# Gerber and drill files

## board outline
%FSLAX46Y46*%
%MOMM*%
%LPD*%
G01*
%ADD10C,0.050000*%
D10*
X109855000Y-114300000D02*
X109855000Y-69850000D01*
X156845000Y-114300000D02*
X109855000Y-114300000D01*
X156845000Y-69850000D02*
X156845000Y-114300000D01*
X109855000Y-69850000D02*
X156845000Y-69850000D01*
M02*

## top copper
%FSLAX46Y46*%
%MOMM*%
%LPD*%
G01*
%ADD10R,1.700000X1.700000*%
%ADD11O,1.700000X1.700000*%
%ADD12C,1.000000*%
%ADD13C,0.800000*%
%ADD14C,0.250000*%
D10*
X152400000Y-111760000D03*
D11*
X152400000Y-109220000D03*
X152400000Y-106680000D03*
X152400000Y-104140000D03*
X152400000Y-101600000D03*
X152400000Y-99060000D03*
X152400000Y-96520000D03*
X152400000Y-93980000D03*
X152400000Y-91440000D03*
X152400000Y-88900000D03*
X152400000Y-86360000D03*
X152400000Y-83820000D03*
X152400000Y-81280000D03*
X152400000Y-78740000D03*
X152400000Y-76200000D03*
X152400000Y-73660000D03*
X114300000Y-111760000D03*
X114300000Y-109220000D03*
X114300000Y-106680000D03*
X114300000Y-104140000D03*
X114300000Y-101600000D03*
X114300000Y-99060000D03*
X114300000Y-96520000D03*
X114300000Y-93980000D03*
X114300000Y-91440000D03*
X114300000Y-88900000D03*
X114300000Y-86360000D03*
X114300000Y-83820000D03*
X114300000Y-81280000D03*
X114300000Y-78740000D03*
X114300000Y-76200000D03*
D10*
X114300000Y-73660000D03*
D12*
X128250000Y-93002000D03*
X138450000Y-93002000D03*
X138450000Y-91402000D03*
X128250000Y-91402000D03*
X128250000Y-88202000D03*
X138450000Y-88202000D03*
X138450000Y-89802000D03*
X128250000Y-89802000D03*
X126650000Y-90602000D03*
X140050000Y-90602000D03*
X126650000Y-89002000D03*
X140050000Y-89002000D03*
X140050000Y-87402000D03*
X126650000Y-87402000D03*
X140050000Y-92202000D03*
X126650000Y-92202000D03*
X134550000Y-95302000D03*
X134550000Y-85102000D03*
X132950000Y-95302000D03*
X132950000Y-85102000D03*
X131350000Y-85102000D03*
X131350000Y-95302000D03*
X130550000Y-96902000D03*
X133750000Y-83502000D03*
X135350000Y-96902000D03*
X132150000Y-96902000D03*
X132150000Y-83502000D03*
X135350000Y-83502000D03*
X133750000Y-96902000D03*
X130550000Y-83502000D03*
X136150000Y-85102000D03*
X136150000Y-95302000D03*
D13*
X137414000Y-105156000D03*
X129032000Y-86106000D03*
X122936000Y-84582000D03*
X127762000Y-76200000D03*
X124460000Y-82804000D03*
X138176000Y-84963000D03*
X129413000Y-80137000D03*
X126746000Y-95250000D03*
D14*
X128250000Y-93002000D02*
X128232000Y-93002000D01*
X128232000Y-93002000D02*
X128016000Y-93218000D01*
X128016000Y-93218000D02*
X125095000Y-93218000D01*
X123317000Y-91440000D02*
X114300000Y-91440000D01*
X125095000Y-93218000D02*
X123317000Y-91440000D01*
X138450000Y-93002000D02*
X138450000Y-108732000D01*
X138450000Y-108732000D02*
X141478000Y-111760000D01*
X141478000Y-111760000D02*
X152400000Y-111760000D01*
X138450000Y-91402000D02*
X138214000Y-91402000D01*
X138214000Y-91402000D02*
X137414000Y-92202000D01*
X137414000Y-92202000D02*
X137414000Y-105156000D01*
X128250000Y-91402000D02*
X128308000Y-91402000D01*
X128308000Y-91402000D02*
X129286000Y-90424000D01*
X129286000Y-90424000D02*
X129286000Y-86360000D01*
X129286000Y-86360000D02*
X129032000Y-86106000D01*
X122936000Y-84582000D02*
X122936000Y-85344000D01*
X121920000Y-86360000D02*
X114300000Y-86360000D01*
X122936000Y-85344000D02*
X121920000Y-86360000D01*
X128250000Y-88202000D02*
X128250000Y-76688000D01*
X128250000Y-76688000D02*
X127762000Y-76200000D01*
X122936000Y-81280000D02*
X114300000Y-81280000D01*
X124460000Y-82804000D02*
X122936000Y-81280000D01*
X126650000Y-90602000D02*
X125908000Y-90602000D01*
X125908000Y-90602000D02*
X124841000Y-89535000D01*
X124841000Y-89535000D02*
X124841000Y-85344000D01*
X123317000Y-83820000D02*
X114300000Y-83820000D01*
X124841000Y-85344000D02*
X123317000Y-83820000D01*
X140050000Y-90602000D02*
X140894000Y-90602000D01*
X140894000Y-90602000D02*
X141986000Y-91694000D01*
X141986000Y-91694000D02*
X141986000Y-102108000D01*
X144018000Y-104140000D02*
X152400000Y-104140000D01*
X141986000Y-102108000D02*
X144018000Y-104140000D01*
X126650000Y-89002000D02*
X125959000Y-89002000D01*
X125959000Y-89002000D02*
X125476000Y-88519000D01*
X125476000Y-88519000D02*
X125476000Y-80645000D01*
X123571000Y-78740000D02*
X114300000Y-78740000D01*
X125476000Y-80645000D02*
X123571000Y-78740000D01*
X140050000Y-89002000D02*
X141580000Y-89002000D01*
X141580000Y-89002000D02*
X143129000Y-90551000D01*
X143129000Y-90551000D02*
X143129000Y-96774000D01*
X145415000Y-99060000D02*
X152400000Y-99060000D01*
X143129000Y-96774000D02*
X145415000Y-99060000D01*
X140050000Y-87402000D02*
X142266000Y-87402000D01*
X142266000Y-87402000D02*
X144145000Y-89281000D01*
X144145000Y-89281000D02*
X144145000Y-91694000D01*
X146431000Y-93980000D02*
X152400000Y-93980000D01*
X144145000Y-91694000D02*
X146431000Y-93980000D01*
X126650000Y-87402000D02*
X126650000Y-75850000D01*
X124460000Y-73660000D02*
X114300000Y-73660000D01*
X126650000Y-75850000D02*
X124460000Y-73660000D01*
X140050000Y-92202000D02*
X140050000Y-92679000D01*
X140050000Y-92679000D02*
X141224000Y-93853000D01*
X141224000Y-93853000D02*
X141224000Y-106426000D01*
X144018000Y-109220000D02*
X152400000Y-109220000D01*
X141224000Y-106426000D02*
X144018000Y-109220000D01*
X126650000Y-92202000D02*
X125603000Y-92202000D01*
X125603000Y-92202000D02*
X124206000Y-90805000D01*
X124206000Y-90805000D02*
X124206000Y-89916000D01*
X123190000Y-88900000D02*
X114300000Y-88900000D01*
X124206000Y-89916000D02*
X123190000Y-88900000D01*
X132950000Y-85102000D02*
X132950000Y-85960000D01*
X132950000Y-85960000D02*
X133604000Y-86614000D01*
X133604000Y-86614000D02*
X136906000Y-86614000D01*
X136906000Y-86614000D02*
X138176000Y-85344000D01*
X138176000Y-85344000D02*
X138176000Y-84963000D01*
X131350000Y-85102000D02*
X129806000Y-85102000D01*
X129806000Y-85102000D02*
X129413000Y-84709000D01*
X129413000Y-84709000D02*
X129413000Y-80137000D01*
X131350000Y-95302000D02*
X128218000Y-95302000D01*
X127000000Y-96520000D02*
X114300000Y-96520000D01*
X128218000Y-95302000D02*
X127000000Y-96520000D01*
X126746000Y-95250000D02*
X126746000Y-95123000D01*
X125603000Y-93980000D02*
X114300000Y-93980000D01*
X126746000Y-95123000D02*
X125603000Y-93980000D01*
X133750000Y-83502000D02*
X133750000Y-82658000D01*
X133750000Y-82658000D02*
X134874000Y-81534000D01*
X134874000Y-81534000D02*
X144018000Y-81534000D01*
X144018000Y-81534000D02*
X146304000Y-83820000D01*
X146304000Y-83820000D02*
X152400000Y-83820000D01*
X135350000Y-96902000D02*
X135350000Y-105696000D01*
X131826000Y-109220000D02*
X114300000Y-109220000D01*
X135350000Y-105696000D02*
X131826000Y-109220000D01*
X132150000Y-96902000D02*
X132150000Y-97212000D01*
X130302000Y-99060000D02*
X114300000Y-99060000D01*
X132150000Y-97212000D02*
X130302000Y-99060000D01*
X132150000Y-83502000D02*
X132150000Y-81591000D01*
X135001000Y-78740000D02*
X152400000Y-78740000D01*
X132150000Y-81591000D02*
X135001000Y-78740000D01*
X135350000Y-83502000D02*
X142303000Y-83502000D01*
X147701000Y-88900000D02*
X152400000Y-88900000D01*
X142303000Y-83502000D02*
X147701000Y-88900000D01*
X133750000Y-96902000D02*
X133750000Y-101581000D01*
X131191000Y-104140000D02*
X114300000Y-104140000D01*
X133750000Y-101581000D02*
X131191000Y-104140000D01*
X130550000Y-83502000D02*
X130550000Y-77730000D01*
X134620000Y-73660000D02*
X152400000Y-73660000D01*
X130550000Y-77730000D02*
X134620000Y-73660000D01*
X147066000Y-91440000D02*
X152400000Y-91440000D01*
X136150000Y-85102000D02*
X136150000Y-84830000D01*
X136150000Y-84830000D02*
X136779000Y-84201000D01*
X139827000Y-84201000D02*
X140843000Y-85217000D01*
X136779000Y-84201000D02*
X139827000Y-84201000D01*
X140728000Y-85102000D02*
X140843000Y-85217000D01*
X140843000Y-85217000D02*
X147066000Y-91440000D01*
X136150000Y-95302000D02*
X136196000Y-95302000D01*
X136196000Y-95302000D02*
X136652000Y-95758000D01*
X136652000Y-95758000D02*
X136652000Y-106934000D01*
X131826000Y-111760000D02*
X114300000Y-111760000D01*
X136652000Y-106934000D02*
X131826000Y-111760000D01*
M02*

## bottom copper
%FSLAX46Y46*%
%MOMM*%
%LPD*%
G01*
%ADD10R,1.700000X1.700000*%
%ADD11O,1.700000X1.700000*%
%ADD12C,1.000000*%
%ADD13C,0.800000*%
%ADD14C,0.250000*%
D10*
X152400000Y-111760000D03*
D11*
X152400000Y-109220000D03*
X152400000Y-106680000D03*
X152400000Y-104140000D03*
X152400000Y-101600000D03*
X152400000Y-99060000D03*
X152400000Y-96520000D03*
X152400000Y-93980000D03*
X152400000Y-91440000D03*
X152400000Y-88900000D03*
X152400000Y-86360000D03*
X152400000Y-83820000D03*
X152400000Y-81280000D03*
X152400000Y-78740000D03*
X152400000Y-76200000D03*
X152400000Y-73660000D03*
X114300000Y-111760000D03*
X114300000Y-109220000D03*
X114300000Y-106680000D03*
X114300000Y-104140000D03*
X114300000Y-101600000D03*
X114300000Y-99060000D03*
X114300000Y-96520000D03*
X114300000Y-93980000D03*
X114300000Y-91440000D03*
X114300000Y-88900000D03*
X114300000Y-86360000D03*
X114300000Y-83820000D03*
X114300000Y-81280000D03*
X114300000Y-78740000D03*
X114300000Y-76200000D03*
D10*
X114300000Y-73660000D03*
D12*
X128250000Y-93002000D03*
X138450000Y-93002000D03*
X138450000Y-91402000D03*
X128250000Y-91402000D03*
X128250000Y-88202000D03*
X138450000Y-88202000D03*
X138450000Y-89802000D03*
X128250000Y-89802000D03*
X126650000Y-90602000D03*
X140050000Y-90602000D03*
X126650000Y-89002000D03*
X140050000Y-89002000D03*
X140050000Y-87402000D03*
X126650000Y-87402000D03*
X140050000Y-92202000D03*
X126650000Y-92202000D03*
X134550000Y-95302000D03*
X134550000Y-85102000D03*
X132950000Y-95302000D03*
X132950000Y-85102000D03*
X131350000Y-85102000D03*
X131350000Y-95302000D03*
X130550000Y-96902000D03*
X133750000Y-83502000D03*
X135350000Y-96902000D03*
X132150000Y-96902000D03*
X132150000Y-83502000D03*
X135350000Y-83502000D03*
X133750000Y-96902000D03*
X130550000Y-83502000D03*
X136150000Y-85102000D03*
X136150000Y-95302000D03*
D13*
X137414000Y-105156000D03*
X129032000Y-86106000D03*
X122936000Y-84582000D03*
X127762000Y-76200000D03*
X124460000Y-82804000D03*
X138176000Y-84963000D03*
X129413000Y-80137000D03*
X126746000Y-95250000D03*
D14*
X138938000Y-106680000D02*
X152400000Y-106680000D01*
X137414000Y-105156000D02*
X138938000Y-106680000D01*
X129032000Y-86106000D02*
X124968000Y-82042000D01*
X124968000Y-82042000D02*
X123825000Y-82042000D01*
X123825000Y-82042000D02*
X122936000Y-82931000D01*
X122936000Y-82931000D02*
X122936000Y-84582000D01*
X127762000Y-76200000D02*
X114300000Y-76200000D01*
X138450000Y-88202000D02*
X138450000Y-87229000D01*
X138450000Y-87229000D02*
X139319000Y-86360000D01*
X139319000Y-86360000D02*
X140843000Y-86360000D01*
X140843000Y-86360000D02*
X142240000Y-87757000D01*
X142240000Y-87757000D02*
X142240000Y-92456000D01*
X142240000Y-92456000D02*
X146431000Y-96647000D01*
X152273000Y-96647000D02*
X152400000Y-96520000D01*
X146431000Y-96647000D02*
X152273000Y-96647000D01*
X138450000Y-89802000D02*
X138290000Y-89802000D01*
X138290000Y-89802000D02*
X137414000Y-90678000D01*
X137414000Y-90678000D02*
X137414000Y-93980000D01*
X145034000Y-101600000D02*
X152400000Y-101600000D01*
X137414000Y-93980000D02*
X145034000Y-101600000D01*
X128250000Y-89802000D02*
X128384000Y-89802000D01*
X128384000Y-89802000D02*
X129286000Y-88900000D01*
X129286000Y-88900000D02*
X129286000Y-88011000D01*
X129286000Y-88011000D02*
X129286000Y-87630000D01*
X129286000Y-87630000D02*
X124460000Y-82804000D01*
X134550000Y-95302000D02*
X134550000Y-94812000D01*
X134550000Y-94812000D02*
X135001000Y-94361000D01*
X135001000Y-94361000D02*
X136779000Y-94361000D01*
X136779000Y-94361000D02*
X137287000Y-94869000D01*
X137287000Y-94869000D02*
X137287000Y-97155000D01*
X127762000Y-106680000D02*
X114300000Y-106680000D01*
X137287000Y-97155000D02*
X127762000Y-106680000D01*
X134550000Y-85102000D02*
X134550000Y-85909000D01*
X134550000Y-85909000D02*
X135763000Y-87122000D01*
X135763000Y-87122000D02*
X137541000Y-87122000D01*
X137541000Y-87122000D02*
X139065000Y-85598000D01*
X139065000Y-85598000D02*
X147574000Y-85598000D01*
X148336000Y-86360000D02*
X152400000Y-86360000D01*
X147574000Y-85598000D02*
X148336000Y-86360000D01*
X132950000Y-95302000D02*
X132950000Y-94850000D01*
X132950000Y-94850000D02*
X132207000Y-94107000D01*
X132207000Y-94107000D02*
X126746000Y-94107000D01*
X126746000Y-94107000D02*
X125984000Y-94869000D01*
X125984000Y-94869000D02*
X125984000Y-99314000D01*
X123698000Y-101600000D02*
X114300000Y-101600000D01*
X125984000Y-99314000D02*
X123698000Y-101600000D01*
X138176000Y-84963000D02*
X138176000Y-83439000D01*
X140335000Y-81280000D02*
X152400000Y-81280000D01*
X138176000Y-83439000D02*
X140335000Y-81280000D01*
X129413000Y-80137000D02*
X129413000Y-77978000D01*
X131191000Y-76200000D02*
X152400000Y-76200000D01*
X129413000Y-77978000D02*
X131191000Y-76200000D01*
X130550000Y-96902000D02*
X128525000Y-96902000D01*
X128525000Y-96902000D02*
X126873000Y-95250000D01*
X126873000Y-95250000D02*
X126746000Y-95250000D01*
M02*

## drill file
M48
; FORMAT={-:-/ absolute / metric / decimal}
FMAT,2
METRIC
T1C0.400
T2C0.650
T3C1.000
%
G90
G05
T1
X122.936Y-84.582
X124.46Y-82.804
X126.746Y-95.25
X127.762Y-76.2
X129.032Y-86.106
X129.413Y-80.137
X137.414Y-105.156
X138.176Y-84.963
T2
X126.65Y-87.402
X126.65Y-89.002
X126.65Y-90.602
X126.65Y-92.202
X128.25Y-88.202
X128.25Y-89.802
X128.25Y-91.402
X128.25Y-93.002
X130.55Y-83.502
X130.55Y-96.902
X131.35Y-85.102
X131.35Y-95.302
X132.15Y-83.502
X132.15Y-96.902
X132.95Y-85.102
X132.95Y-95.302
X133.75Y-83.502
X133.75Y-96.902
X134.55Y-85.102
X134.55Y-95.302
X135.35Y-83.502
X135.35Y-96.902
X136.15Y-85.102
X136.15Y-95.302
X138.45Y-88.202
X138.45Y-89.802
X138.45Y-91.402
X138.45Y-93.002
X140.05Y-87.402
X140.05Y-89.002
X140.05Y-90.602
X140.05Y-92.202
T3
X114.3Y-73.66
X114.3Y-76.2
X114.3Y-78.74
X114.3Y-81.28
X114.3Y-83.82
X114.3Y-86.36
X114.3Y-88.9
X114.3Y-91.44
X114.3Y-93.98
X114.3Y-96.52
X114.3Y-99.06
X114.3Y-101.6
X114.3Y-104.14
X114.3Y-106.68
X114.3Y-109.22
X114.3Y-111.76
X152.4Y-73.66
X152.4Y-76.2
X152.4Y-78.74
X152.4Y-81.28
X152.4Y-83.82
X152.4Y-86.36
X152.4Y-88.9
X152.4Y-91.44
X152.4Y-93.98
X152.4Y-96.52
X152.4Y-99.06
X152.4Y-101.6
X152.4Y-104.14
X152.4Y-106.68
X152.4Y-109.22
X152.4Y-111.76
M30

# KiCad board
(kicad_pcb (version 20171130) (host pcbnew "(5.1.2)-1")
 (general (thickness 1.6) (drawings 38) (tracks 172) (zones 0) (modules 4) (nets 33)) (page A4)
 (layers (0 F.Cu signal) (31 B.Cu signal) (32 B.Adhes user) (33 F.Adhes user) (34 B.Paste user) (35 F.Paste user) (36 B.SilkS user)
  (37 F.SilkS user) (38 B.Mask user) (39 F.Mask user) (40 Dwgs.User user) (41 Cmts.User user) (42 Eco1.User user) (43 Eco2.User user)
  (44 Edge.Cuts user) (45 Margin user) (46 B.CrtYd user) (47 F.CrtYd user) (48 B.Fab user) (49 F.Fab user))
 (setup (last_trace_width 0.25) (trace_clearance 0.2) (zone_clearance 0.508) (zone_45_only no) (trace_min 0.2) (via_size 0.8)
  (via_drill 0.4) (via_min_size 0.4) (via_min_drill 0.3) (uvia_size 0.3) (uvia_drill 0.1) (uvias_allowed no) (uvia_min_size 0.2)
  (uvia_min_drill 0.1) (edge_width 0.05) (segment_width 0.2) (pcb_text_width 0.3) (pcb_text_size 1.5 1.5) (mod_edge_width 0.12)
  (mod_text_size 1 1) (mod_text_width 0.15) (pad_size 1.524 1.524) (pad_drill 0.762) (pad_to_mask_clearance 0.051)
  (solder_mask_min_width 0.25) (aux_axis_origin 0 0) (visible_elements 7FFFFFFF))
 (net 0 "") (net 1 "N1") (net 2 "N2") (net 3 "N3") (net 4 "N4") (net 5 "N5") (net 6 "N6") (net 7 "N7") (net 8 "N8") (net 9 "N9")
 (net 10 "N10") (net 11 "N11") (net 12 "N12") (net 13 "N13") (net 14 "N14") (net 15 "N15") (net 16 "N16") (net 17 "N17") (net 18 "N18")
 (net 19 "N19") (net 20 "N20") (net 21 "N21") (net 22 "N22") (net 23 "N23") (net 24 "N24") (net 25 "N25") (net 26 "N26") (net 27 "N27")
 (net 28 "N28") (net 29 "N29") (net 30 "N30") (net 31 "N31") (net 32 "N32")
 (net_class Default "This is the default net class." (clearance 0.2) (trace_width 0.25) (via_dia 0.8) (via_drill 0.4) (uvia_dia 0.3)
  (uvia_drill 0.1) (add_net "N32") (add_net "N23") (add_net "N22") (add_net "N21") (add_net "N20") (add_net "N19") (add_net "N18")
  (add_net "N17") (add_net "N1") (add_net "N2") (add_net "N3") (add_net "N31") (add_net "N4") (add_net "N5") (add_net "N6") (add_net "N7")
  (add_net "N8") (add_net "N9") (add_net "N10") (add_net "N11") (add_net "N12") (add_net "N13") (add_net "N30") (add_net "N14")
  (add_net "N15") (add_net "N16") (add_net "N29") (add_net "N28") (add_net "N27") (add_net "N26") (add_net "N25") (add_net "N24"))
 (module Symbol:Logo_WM (layer F.Cu) (at 121.92 109.855)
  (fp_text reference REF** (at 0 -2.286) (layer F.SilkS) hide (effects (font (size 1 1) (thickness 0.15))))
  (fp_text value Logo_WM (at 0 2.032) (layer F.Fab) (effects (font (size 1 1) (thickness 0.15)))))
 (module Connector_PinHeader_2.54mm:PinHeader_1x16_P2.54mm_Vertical (layer B.Cu) (at 152.4 111.76)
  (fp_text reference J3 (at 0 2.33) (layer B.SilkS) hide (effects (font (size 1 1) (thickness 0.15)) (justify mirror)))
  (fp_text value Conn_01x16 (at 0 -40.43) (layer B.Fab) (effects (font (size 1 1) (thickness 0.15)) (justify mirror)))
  (pad 1 thru_hole rect (at 0 0) (size 1.7 1.7) (drill 1) (layers *.Cu *.Mask) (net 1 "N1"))
  (pad 2 thru_hole oval (at 0 -2.54) (size 1.7 1.7) (drill 1) (layers *.Cu *.Mask) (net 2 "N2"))
  (pad 3 thru_hole oval (at 0 -5.08) (size 1.7 1.7) (drill 1) (layers *.Cu *.Mask) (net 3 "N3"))
  (pad 4 thru_hole oval (at 0 -7.62) (size 1.7 1.7) (drill 1) (layers *.Cu *.Mask) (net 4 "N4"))
  (pad 5 thru_hole oval (at 0 -10.16) (size 1.7 1.7) (drill 1) (layers *.Cu *.Mask) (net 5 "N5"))
  (pad 6 thru_hole oval (at 0 -12.7) (size 1.7 1.7) (drill 1) (layers *.Cu *.Mask) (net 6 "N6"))
  (pad 7 thru_hole oval (at 0 -15.24) (size 1.7 1.7) (drill 1) (layers *.Cu *.Mask) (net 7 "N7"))
  (pad 8 thru_hole oval (at 0 -17.78) (size 1.7 1.7) (drill 1) (layers *.Cu *.Mask) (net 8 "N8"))
  (pad 9 thru_hole oval (at 0 -20.32) (size 1.7 1.7) (drill 1) (layers *.Cu *.Mask) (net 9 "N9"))
  (pad 10 thru_hole oval (at 0 -22.86) (size 1.7 1.7) (drill 1) (layers *.Cu *.Mask) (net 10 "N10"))
  (pad 11 thru_hole oval (at 0 -25.4) (size 1.7 1.7) (drill 1) (layers *.Cu *.Mask) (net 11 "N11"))
  (pad 12 thru_hole oval (at 0 -27.94) (size 1.7 1.7) (drill 1) (layers *.Cu *.Mask) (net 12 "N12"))
  (pad 13 thru_hole oval (at 0 -30.48) (size 1.7 1.7) (drill 1) (layers *.Cu *.Mask) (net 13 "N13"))
  (pad 14 thru_hole oval (at 0 -33.02) (size 1.7 1.7) (drill 1) (layers *.Cu *.Mask) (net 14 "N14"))
  (pad 15 thru_hole oval (at 0 -35.56) (size 1.7 1.7) (drill 1) (layers *.Cu *.Mask) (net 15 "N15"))
  (pad 16 thru_hole oval (at 0 -38.1) (size 1.7 1.7) (drill 1) (layers *.Cu *.Mask) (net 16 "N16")))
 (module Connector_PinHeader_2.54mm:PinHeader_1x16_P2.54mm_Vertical (layer B.Cu) (at 114.3 73.66 180)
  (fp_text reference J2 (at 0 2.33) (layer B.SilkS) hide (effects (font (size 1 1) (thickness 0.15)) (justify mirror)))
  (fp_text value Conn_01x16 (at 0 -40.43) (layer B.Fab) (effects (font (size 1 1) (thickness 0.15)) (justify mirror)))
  (pad 16 thru_hole oval (at 0 -38.1 180) (size 1.7 1.7) (drill 1) (layers *.Cu *.Mask) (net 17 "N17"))
  (pad 15 thru_hole oval (at 0 -35.56 180) (size 1.7 1.7) (drill 1) (layers *.Cu *.Mask) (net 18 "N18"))
  (pad 14 thru_hole oval (at 0 -33.02 180) (size 1.7 1.7) (drill 1) (layers *.Cu *.Mask) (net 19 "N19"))
  (pad 13 thru_hole oval (at 0 -30.48 180) (size 1.7 1.7) (drill 1) (layers *.Cu *.Mask) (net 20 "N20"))
  (pad 12 thru_hole oval (at 0 -27.94 180) (size 1.7 1.7) (drill 1) (layers *.Cu *.Mask) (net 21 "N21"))
  (pad 11 thru_hole oval (at 0 -25.4 180) (size 1.7 1.7) (drill 1) (layers *.Cu *.Mask) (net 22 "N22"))
  (pad 10 thru_hole oval (at 0 -22.86 180) (size 1.7 1.7) (drill 1) (layers *.Cu *.Mask) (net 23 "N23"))
  (pad 9 thru_hole oval (at 0 -20.32 180) (size 1.7 1.7) (drill 1) (layers *.Cu *.Mask) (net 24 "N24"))
  (pad 8 thru_hole oval (at 0 -17.78 180) (size 1.7 1.7) (drill 1) (layers *.Cu *.Mask) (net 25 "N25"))
  (pad 7 thru_hole oval (at 0 -15.24 180) (size 1.7 1.7) (drill 1) (layers *.Cu *.Mask) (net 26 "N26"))
  (pad 6 thru_hole oval (at 0 -12.7 180) (size 1.7 1.7) (drill 1) (layers *.Cu *.Mask) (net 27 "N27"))
  (pad 5 thru_hole oval (at 0 -10.16 180) (size 1.7 1.7) (drill 1) (layers *.Cu *.Mask) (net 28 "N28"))
  (pad 4 thru_hole oval (at 0 -7.62 180) (size 1.7 1.7) (drill 1) (layers *.Cu *.Mask) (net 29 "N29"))
  (pad 3 thru_hole oval (at 0 -5.08 180) (size 1.7 1.7) (drill 1) (layers *.Cu *.Mask) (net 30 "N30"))
  (pad 2 thru_hole oval (at 0 -2.54 180) (size 1.7 1.7) (drill 1) (layers *.Cu *.Mask) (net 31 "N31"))
  (pad 1 thru_hole rect (at 0 0 180) (size 1.7 1.7) (drill 1) (layers *.Cu *.Mask) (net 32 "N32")))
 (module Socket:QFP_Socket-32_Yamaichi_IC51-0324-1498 (layer F.Cu) (at 133.35 92.202)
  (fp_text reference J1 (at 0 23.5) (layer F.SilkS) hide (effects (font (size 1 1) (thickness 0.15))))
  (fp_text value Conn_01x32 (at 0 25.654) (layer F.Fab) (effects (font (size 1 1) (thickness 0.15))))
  (pad 8 thru_hole circle (at -5.1 0.8) (size 1 1) (drill 0.65) (layers *.Cu *.Mask) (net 25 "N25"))
  (pad 17 thru_hole circle (at 5.1 0.8) (size 1 1) (drill 0.65) (layers *.Cu *.Mask) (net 1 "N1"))
  (pad 19 thru_hole circle (at 5.1 -0.8) (size 1 1) (drill 0.65) (layers *.Cu *.Mask) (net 3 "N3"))
  (pad 6 thru_hole circle (at -5.1 -0.8) (size 1 1) (drill 0.65) (layers *.Cu *.Mask) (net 27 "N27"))
  (pad 2 thru_hole circle (at -5.1 -4) (size 1 1) (drill 0.65) (layers *.Cu *.Mask) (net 31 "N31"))
  (pad 23 thru_hole circle (at 5.1 -4) (size 1 1) (drill 0.65) (layers *.Cu *.Mask) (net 7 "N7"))
  (pad 21 thru_hole circle (at 5.1 -2.4) (size 1 1) (drill 0.65) (layers *.Cu *.Mask) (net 5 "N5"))
  (pad 4 thru_hole circle (at -5.1 -2.4) (size 1 1) (drill 0.65) (layers *.Cu *.Mask) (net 29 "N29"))
  (pad 5 thru_hole circle (at -6.7 -1.6) (size 1 1) (drill 0.65) (layers *.Cu *.Mask) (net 28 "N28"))
  (pad 20 thru_hole circle (at 6.7 -1.6) (size 1 1) (drill 0.65) (layers *.Cu *.Mask) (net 4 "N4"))
  (pad 3 thru_hole circle (at -6.7 -3.2) (size 1 1) (drill 0.65) (layers *.Cu *.Mask) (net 30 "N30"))
  (pad 22 thru_hole circle (at 6.7 -3.2) (size 1 1) (drill 0.65) (layers *.Cu *.Mask) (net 6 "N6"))
  (pad 24 thru_hole circle (at 6.7 -4.8) (size 1 1) (drill 0.65) (layers *.Cu *.Mask) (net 8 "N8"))
  (pad 1 thru_hole circle (at -6.7 -4.8) (size 1 1) (drill 0.65) (layers *.Cu *.Mask) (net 32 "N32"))
  (pad 18 thru_hole circle (at 6.7 0) (size 1 1) (drill 0.65) (layers *.Cu *.Mask) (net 2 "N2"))
  (pad 7 thru_hole circle (at -6.7 0) (size 1 1) (drill 0.65) (layers *.Cu *.Mask) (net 26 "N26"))
  (pad 14 thru_hole circle (at 1.2 3.1 90) (size 1 1) (drill 0.65) (layers *.Cu *.Mask) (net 19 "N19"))
  (pad 27 thru_hole circle (at 1.2 -7.1 90) (size 1 1) (drill 0.65) (layers *.Cu *.Mask) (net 11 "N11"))
  (pad 12 thru_hole circle (at -0.4 3.1 90) (size 1 1) (drill 0.65) (layers *.Cu *.Mask) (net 21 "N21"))
  (pad 29 thru_hole circle (at -0.4 -7.1 90) (size 1 1) (drill 0.65) (layers *.Cu *.Mask) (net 13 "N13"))
  (pad 31 thru_hole circle (at -2 -7.1 90) (size 1 1) (drill 0.65) (layers *.Cu *.Mask) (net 15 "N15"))
  (pad 10 thru_hole circle (at -2 3.1 90) (size 1 1) (drill 0.65) (layers *.Cu *.Mask) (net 23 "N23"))
  (pad 9 thru_hole circle (at -2.8 4.7 90) (size 1 1) (drill 0.65) (layers *.Cu *.Mask) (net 24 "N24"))
  (pad 28 thru_hole circle (at 0.4 -8.7 90) (size 1 1) (drill 0.65) (layers *.Cu *.Mask) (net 12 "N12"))
  (pad 15 thru_hole circle (at 2 4.7 90) (size 1 1) (drill 0.65) (layers *.Cu *.Mask) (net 18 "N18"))
  (pad 11 thru_hole circle (at -1.2 4.7 90) (size 1 1) (drill 0.65) (layers *.Cu *.Mask) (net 22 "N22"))
  (pad 30 thru_hole circle (at -1.2 -8.7 90) (size 1 1) (drill 0.65) (layers *.Cu *.Mask) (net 14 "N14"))
  (pad 26 thru_hole circle (at 2 -8.7 90) (size 1 1) (drill 0.65) (layers *.Cu *.Mask) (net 10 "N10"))
  (pad 13 thru_hole circle (at 0.4 4.7 90) (size 1 1) (drill 0.65) (layers *.Cu *.Mask) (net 20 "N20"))
  (pad 32 thru_hole circle (at -2.8 -8.7 90) (size 1 1) (drill 0.65) (layers *.Cu *.Mask) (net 16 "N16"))
  (pad 25 thru_hole circle (at 2.8 -7.1 90) (size 1 1) (drill 0.65) (layers *.Cu *.Mask) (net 9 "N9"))
  (pad 16 thru_hole circle (at 2.8 3.1 90) (size 1 1) (drill 0.65) (layers *.Cu *.Mask) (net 17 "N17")))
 (gr_line (start 109.855 114.3) (end 109.855 69.85) (layer Edge.Cuts) (width 0.05))
 (gr_line (start 156.845 114.3) (end 109.855 114.3) (layer Edge.Cuts) (width 0.05))
 (gr_line (start 156.845 69.85) (end 156.845 114.3) (layer Edge.Cuts) (width 0.05))
 (gr_line (start 109.855 69.85) (end 156.845 69.85) (layer Edge.Cuts) (width 0.05))
 (segment (start 128.25 93.002) (end 128.232 93.002) (width 0.25) (layer F.Cu) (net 25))
 (segment (start 128.232 93.002) (end 128.016 93.218) (width 0.25) (layer F.Cu) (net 25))
 (segment (start 128.016 93.218) (end 125.095 93.218) (width 0.25) (layer F.Cu) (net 25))
 (segment (start 123.317 91.44) (end 114.3 91.44) (width 0.25) (layer F.Cu) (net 25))
 (segment (start 125.095 93.218) (end 123.317 91.44) (width 0.25) (layer F.Cu) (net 25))
 (segment (start 138.45 93.002) (end 138.45 108.732) (width 0.25) (layer F.Cu) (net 1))
 (segment (start 138.45 108.732) (end 141.478 111.76) (width 0.25) (layer F.Cu) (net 1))
 (segment (start 141.478 111.76) (end 152.4 111.76) (width 0.25) (layer F.Cu) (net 1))
 (segment (start 138.45 91.402) (end 138.214 91.402) (width 0.25) (layer F.Cu) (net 3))
 (segment (start 138.214 91.402) (end 137.414 92.202) (width 0.25) (layer F.Cu) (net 3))
 (via (at 137.414 105.156) (size 0.8) (drill 0.4) (layers F.Cu B.Cu) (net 3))
 (segment (start 137.414 92.202) (end 137.414 105.156) (width 0.25) (layer F.Cu) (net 3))
 (segment (start 138.938 106.68) (end 152.4 106.68) (width 0.25) (layer B.Cu) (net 3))
 (segment (start 137.414 105.156) (end 138.938 106.68) (width 0.25) (layer B.Cu) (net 3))
 (segment (start 128.25 91.402) (end 128.308 91.402) (width 0.25) (layer F.Cu) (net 27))
 (segment (start 128.308 91.402) (end 129.286 90.424) (width 0.25) (layer F.Cu) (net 27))
 (via (at 129.032 86.106) (size 0.8) (drill 0.4) (layers F.Cu B.Cu) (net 27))
 (segment (start 129.286 90.424) (end 129.286 86.36) (width 0.25) (layer F.Cu) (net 27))
 (segment (start 129.286 86.36) (end 129.032 86.106) (width 0.25) (layer F.Cu) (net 27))
 (segment (start 129.032 86.106) (end 124.968 82.042) (width 0.25) (layer B.Cu) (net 27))
 (segment (start 124.968 82.042) (end 123.825 82.042) (width 0.25) (layer B.Cu) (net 27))
 (via (at 122.936 84.582) (size 0.8) (drill 0.4) (layers F.Cu B.Cu) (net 27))
 (segment (start 123.825 82.042) (end 122.936 82.931) (width 0.25) (layer B.Cu) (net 27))
 (segment (start 122.936 82.931) (end 122.936 84.582) (width 0.25) (layer B.Cu) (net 27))
 (segment (start 122.936 84.582) (end 122.936 85.344) (width 0.25) (layer F.Cu) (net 27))
 (segment (start 121.92 86.36) (end 114.3 86.36) (width 0.25) (layer F.Cu) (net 27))
 (segment (start 122.936 85.344) (end 121.92 86.36) (width 0.25) (layer F.Cu) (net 27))
 (via (at 127.762 76.2) (size 0.8) (drill 0.4) (layers F.Cu B.Cu) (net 31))
 (segment (start 128.25 88.202) (end 128.25 76.688) (width 0.25) (layer F.Cu) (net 31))
 (segment (start 128.25 76.688) (end 127.762 76.2) (width 0.25) (layer F.Cu) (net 31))
 (segment (start 127.762 76.2) (end 114.3 76.2) (width 0.25) (layer B.Cu) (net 31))
 (segment (start 138.45 88.202) (end 138.45 87.229) (width 0.25) (layer B.Cu) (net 7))
 (segment (start 138.45 87.229) (end 139.319 86.36) (width 0.25) (layer B.Cu) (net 7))
 (segment (start 139.319 86.36) (end 140.843 86.36) (width 0.25) (layer B.Cu) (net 7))
 (segment (start 140.843 86.36) (end 142.24 87.757) (width 0.25) (layer B.Cu) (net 7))
 (segment (start 142.24 87.757) (end 142.24 92.456) (width 0.25) (layer B.Cu) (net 7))
 (segment (start 142.24 92.456) (end 146.431 96.647) (width 0.25) (layer B.Cu) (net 7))
 (segment (start 152.273 96.647) (end 152.4 96.52) (width 0.25) (layer B.Cu) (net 7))
 (segment (start 146.431 96.647) (end 152.273 96.647) (width 0.25) (layer B.Cu) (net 7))
 (segment (start 138.45 89.802) (end 138.29 89.802) (width 0.25) (layer B.Cu) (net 5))
 (segment (start 138.29 89.802) (end 137.414 90.678) (width 0.25) (layer B.Cu) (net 5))
 (segment (start 137.414 90.678) (end 137.414 93.98) (width 0.25) (layer B.Cu) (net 5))
 (segment (start 145.034 101.6) (end 152.4 101.6) (width 0.25) (layer B.Cu) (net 5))
 (segment (start 137.414 93.98) (end 145.034 101.6) (width 0.25) (layer B.Cu) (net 5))
 (segment (start 128.25 89.802) (end 128.384 89.802) (width 0.25) (layer B.Cu) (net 29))
 (segment (start 128.384 89.802) (end 129.286 88.9) (width 0.25) (layer B.Cu) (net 29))
 (segment (start 129.286 88.9) (end 129.286 88.011) (width 0.25) (layer B.Cu) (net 29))
 (via (at 124.46 82.804) (size 0.8) (drill 0.4) (layers F.Cu B.Cu) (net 29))
 (segment (start 129.286 88.011) (end 129.286 87.63) (width 0.25) (layer B.Cu) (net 29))
 (segment (start 129.286 87.63) (end 124.46 82.804) (width 0.25) (layer B.Cu) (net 29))
 (segment (start 122.936 81.28) (end 114.3 81.28) (width 0.25) (layer F.Cu) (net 29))
 (segment (start 124.46 82.804) (end 122.936 81.28) (width 0.25) (layer F.Cu) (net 29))
 (segment (start 126.65 90.602) (end 125.908 90.602) (width 0.25) (layer F.Cu) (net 28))
 (segment (start 125.908 90.602) (end 124.841 89.535) (width 0.25) (layer F.Cu) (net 28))
 (segment (start 124.841 89.535) (end 124.841 85.344) (width 0.25) (layer F.Cu) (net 28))
 (segment (start 123.317 83.82) (end 114.3 83.82) (width 0.25) (layer F.Cu) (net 28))
 (segment (start 124.841 85.344) (end 123.317 83.82) (width 0.25) (layer F.Cu) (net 28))
 (segment (start 140.05 90.602) (end 140.894 90.602) (width 0.25) (layer F.Cu) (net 4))
 (segment (start 140.894 90.602) (end 141.986 91.694) (width 0.25) (layer F.Cu) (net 4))
 (segment (start 141.986 91.694) (end 141.986 102.108) (width 0.25) (layer F.Cu) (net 4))
 (segment (start 144.018 104.14) (end 152.4 104.14) (width 0.25) (layer F.Cu) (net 4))
 (segment (start 141.986 102.108) (end 144.018 104.14) (width 0.25) (layer F.Cu) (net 4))
 (segment (start 126.65 89.002) (end 125.959 89.002) (width 0.25) (layer F.Cu) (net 30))
 (segment (start 125.959 89.002) (end 125.476 88.519) (width 0.25) (layer F.Cu) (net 30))
 (segment (start 125.476 88.519) (end 125.476 80.645) (width 0.25) (layer F.Cu) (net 30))
 (segment (start 123.571 78.74) (end 114.3 78.74) (width 0.25) (layer F.Cu) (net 30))
 (segment (start 125.476 80.645) (end 123.571 78.74) (width 0.25) (layer F.Cu) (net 30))
 (segment (start 140.05 89.002) (end 141.58 89.002) (width 0.25) (layer F.Cu) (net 6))
 (segment (start 141.58 89.002) (end 143.129 90.551) (width 0.25) (layer F.Cu) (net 6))
 (segment (start 143.129 90.551) (end 143.129 96.774) (width 0.25) (layer F.Cu) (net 6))
 (segment (start 145.415 99.06) (end 152.4 99.06) (width 0.25) (layer F.Cu) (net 6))
 (segment (start 143.129 96.774) (end 145.415 99.06) (width 0.25) (layer F.Cu) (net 6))
 (segment (start 140.05 87.402) (end 142.266 87.402) (width 0.25) (layer F.Cu) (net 8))
 (segment (start 142.266 87.402) (end 144.145 89.281) (width 0.25) (layer F.Cu) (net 8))
 (segment (start 144.145 89.281) (end 144.145 91.694) (width 0.25) (layer F.Cu) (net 8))
 (segment (start 146.431 93.98) (end 152.4 93.98) (width 0.25) (layer F.Cu) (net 8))
 (segment (start 144.145 91.694) (end 146.431 93.98) (width 0.25) (layer F.Cu) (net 8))
 (segment (start 126.65 87.402) (end 126.65 75.85) (width 0.25) (layer F.Cu) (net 32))
 (segment (start 124.46 73.66) (end 114.3 73.66) (width 0.25) (layer F.Cu) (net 32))
 (segment (start 126.65 75.85) (end 124.46 73.66) (width 0.25) (layer F.Cu) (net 32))
 (segment (start 140.05 92.202) (end 140.05 92.679) (width 0.25) (layer F.Cu) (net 2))
 (segment (start 140.05 92.679) (end 141.224 93.853) (width 0.25) (layer F.Cu) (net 2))
 (segment (start 141.224 93.853) (end 141.224 106.426) (width 0.25) (layer F.Cu) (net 2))
 (segment (start 144.018 109.22) (end 152.4 109.22) (width 0.25) (layer F.Cu) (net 2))
 (segment (start 141.224 106.426) (end 144.018 109.22) (width 0.25) (layer F.Cu) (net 2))
 (segment (start 126.65 92.202) (end 125.603 92.202) (width 0.25) (layer F.Cu) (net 26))
 (segment (start 125.603 92.202) (end 124.206 90.805) (width 0.25) (layer F.Cu) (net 26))
 (segment (start 124.206 90.805) (end 124.206 89.916) (width 0.25) (layer F.Cu) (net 26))
 (segment (start 123.19 88.9) (end 114.3 88.9) (width 0.25) (layer F.Cu) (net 26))
 (segment (start 124.206 89.916) (end 123.19 88.9) (width 0.25) (layer F.Cu) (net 26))
 (segment (start 134.55 95.302) (end 134.55 94.812) (width 0.25) (layer B.Cu) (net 19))
 (segment (start 134.55 94.812) (end 135.001 94.361) (width 0.25) (layer B.Cu) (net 19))
 (segment (start 135.001 94.361) (end 136.779 94.361) (width 0.25) (layer B.Cu) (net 19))
 (segment (start 136.779 94.361) (end 137.287 94.869) (width 0.25) (layer B.Cu) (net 19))
 (segment (start 137.287 94.869) (end 137.287 97.155) (width 0.25) (layer B.Cu) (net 19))
 (segment (start 127.762 106.68) (end 114.3 106.68) (width 0.25) (layer B.Cu) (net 19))
 (segment (start 137.287 97.155) (end 127.762 106.68) (width 0.25) (layer B.Cu) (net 19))
 (segment (start 134.55 85.102) (end 134.55 85.909) (width 0.25) (layer B.Cu) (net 11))
 (segment (start 134.55 85.909) (end 135.763 87.122) (width 0.25) (layer B.Cu) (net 11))
 (segment (start 135.763 87.122) (end 137.541 87.122) (width 0.25) (layer B.Cu) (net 11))
 (segment (start 137.541 87.122) (end 139.065 85.598) (width 0.25) (layer B.Cu) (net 11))
 (segment (start 139.065 85.598) (end 147.574 85.598) (width 0.25) (layer B.Cu) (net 11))
 (segment (start 148.336 86.36) (end 152.4 86.36) (width 0.25) (layer B.Cu) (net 11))
 (segment (start 147.574 85.598) (end 148.336 86.36) (width 0.25) (layer B.Cu) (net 11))
 (segment (start 132.95 95.302) (end 132.95 94.85) (width 0.25) (layer B.Cu) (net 21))
 (segment (start 132.95 94.85) (end 132.207 94.107) (width 0.25) (layer B.Cu) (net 21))
 (segment (start 132.207 94.107) (end 126.746 94.107) (width 0.25) (layer B.Cu) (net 21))
 (segment (start 126.746 94.107) (end 125.984 94.869) (width 0.25) (layer B.Cu) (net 21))
 (segment (start 125.984 94.869) (end 125.984 99.314) (width 0.25) (layer B.Cu) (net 21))
 (segment (start 123.698 101.6) (end 114.3 101.6) (width 0.25) (layer B.Cu) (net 21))
 (segment (start 125.984 99.314) (end 123.698 101.6) (width 0.25) (layer B.Cu) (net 21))
 (segment (start 132.95 85.102) (end 132.95 85.96) (width 0.25) (layer F.Cu) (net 13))
 (segment (start 132.95 85.96) (end 133.604 86.614) (width 0.25) (layer F.Cu) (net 13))
 (segment (start 133.604 86.614) (end 136.906 86.614) (width 0.25) (layer F.Cu) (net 13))
 (via (at 138.176 84.963) (size 0.8) (drill 0.4) (layers F.Cu B.Cu) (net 13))
 (segment (start 136.906 86.614) (end 138.176 85.344) (width 0.25) (layer F.Cu) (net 13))
 (segment (start 138.176 85.344) (end 138.176 84.963) (width 0.25) (layer F.Cu) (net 13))
 (segment (start 138.176 84.963) (end 138.176 83.439) (width 0.25) (layer B.Cu) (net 13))
 (segment (start 140.335 81.28) (end 152.4 81.28) (width 0.25) (layer B.Cu) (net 13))
 (segment (start 138.176 83.439) (end 140.335 81.28) (width 0.25) (layer B.Cu) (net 13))
 (segment (start 131.35 85.102) (end 129.806 85.102) (width 0.25) (layer F.Cu) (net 15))
 (via (at 129.413 80.137) (size 0.8) (drill 0.4) (layers F.Cu B.Cu) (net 15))
 (segment (start 129.806 85.102) (end 129.413 84.709) (width 0.25) (layer F.Cu) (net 15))
 (segment (start 129.413 84.709) (end 129.413 80.137) (width 0.25) (layer F.Cu) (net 15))
 (segment (start 129.413 80.137) (end 129.413 77.978) (width 0.25) (layer B.Cu) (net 15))
 (segment (start 131.191 76.2) (end 152.4 76.2) (width 0.25) (layer B.Cu) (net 15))
 (segment (start 129.413 77.978) (end 131.191 76.2) (width 0.25) (layer B.Cu) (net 15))
 (segment (start 131.35 95.302) (end 128.218 95.302) (width 0.25) (layer F.Cu) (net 23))
 (segment (start 127 96.52) (end 114.3 96.52) (width 0.25) (layer F.Cu) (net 23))
 (segment (start 128.218 95.302) (end 127 96.52) (width 0.25) (layer F.Cu) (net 23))
 (segment (start 130.55 96.902) (end 128.525 96.902) (width 0.25) (layer B.Cu) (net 24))
 (via (at 126.746 95.25) (size 0.8) (drill 0.4) (layers F.Cu B.Cu) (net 24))
 (segment (start 128.525 96.902) (end 126.873 95.25) (width 0.25) (layer B.Cu) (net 24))
 (segment (start 126.873 95.25) (end 126.746 95.25) (width 0.25) (layer B.Cu) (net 24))
 (segment (start 126.746 95.25) (end 126.746 95.123) (width 0.25) (layer F.Cu) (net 24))
 (segment (start 125.603 93.98) (end 114.3 93.98) (width 0.25) (layer F.Cu) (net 24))
 (segment (start 126.746 95.123) (end 125.603 93.98) (width 0.25) (layer F.Cu) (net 24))
 (segment (start 133.75 83.502) (end 133.75 82.658) (width 0.25) (layer F.Cu) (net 12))
 (segment (start 133.75 82.658) (end 134.874 81.534) (width 0.25) (layer F.Cu) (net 12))
 (segment (start 134.874 81.534) (end 144.018 81.534) (width 0.25) (layer F.Cu) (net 12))
 (segment (start 144.018 81.534) (end 146.304 83.82) (width 0.25) (layer F.Cu) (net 12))
 (segment (start 146.304 83.82) (end 152.4 83.82) (width 0.25) (layer F.Cu) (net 12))
 (segment (start 135.35 96.902) (end 135.35 105.696) (width 0.25) (layer F.Cu) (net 18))
 (segment (start 131.826 109.22) (end 114.3 109.22) (width 0.25) (layer F.Cu) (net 18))
 (segment (start 135.35 105.696) (end 131.826 109.22) (width 0.25) (layer F.Cu) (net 18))
 (segment (start 132.15 96.902) (end 132.15 97.212) (width 0.25) (layer F.Cu) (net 22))
 (segment (start 130.302 99.06) (end 114.3 99.06) (width 0.25) (layer F.Cu) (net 22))
 (segment (start 132.15 97.212) (end 130.302 99.06) (width 0.25) (layer F.Cu) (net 22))
 (segment (start 132.15 83.502) (end 132.15 81.591) (width 0.25) (layer F.Cu) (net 14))
 (segment (start 135.001 78.74) (end 152.4 78.74) (width 0.25) (layer F.Cu) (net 14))
 (segment (start 132.15 81.591) (end 135.001 78.74) (width 0.25) (layer F.Cu) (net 14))
 (segment (start 135.35 83.502) (end 142.303 83.502) (width 0.25) (layer F.Cu) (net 10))
 (segment (start 147.701 88.9) (end 152.4 88.9) (width 0.25) (layer F.Cu) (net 10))
 (segment (start 142.303 83.502) (end 147.701 88.9) (width 0.25) (layer F.Cu) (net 10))
 (segment (start 133.75 96.902) (end 133.75 101.581) (width 0.25) (layer F.Cu) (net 20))
 (segment (start 131.191 104.14) (end 114.3 104.14) (width 0.25) (layer F.Cu) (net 20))
 (segment (start 133.75 101.581) (end 131.191 104.14) (width 0.25) (layer F.Cu) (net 20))
 (segment (start 130.55 83.502) (end 130.55 77.73) (width 0.25) (layer F.Cu) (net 16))
 (segment (start 134.62 73.66) (end 152.4 73.66) (width 0.25) (layer F.Cu) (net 16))
 (segment (start 130.55 77.73) (end 134.62 73.66) (width 0.25) (layer F.Cu) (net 16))
 (segment (start 147.066 91.44) (end 152.4 91.44) (width 0.25) (layer F.Cu) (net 9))
 (segment (start 136.15 85.102) (end 136.15 84.83) (width 0.25) (layer F.Cu) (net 9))
 (segment (start 136.15 84.83) (end 136.779 84.201) (width 0.25) (layer F.Cu) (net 9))
 (segment (start 139.827 84.201) (end 140.843 85.217) (width 0.25) (layer F.Cu) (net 9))
 (segment (start 136.779 84.201) (end 139.827 84.201) (width 0.25) (layer F.Cu) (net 9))
 (segment (start 140.728 85.102) (end 140.843 85.217) (width 0.25) (layer F.Cu) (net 9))
 (segment (start 140.843 85.217) (end 147.066 91.44) (width 0.25) (layer F.Cu) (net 9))
 (segment (start 136.15 95.302) (end 136.196 95.302) (width 0.25) (layer F.Cu) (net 17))
 (segment (start 136.196 95.302) (end 136.652 95.758) (width 0.25) (layer F.Cu) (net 17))
 (segment (start 136.652 95.758) (end 136.652 106.934) (width 0.25) (layer F.Cu) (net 17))
 (segment (start 131.826 111.76) (end 114.3 111.76) (width 0.25) (layer F.Cu) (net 17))
 (segment (start 136.652 106.934) (end 131.826 111.76) (width 0.25) (layer F.Cu) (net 17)))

